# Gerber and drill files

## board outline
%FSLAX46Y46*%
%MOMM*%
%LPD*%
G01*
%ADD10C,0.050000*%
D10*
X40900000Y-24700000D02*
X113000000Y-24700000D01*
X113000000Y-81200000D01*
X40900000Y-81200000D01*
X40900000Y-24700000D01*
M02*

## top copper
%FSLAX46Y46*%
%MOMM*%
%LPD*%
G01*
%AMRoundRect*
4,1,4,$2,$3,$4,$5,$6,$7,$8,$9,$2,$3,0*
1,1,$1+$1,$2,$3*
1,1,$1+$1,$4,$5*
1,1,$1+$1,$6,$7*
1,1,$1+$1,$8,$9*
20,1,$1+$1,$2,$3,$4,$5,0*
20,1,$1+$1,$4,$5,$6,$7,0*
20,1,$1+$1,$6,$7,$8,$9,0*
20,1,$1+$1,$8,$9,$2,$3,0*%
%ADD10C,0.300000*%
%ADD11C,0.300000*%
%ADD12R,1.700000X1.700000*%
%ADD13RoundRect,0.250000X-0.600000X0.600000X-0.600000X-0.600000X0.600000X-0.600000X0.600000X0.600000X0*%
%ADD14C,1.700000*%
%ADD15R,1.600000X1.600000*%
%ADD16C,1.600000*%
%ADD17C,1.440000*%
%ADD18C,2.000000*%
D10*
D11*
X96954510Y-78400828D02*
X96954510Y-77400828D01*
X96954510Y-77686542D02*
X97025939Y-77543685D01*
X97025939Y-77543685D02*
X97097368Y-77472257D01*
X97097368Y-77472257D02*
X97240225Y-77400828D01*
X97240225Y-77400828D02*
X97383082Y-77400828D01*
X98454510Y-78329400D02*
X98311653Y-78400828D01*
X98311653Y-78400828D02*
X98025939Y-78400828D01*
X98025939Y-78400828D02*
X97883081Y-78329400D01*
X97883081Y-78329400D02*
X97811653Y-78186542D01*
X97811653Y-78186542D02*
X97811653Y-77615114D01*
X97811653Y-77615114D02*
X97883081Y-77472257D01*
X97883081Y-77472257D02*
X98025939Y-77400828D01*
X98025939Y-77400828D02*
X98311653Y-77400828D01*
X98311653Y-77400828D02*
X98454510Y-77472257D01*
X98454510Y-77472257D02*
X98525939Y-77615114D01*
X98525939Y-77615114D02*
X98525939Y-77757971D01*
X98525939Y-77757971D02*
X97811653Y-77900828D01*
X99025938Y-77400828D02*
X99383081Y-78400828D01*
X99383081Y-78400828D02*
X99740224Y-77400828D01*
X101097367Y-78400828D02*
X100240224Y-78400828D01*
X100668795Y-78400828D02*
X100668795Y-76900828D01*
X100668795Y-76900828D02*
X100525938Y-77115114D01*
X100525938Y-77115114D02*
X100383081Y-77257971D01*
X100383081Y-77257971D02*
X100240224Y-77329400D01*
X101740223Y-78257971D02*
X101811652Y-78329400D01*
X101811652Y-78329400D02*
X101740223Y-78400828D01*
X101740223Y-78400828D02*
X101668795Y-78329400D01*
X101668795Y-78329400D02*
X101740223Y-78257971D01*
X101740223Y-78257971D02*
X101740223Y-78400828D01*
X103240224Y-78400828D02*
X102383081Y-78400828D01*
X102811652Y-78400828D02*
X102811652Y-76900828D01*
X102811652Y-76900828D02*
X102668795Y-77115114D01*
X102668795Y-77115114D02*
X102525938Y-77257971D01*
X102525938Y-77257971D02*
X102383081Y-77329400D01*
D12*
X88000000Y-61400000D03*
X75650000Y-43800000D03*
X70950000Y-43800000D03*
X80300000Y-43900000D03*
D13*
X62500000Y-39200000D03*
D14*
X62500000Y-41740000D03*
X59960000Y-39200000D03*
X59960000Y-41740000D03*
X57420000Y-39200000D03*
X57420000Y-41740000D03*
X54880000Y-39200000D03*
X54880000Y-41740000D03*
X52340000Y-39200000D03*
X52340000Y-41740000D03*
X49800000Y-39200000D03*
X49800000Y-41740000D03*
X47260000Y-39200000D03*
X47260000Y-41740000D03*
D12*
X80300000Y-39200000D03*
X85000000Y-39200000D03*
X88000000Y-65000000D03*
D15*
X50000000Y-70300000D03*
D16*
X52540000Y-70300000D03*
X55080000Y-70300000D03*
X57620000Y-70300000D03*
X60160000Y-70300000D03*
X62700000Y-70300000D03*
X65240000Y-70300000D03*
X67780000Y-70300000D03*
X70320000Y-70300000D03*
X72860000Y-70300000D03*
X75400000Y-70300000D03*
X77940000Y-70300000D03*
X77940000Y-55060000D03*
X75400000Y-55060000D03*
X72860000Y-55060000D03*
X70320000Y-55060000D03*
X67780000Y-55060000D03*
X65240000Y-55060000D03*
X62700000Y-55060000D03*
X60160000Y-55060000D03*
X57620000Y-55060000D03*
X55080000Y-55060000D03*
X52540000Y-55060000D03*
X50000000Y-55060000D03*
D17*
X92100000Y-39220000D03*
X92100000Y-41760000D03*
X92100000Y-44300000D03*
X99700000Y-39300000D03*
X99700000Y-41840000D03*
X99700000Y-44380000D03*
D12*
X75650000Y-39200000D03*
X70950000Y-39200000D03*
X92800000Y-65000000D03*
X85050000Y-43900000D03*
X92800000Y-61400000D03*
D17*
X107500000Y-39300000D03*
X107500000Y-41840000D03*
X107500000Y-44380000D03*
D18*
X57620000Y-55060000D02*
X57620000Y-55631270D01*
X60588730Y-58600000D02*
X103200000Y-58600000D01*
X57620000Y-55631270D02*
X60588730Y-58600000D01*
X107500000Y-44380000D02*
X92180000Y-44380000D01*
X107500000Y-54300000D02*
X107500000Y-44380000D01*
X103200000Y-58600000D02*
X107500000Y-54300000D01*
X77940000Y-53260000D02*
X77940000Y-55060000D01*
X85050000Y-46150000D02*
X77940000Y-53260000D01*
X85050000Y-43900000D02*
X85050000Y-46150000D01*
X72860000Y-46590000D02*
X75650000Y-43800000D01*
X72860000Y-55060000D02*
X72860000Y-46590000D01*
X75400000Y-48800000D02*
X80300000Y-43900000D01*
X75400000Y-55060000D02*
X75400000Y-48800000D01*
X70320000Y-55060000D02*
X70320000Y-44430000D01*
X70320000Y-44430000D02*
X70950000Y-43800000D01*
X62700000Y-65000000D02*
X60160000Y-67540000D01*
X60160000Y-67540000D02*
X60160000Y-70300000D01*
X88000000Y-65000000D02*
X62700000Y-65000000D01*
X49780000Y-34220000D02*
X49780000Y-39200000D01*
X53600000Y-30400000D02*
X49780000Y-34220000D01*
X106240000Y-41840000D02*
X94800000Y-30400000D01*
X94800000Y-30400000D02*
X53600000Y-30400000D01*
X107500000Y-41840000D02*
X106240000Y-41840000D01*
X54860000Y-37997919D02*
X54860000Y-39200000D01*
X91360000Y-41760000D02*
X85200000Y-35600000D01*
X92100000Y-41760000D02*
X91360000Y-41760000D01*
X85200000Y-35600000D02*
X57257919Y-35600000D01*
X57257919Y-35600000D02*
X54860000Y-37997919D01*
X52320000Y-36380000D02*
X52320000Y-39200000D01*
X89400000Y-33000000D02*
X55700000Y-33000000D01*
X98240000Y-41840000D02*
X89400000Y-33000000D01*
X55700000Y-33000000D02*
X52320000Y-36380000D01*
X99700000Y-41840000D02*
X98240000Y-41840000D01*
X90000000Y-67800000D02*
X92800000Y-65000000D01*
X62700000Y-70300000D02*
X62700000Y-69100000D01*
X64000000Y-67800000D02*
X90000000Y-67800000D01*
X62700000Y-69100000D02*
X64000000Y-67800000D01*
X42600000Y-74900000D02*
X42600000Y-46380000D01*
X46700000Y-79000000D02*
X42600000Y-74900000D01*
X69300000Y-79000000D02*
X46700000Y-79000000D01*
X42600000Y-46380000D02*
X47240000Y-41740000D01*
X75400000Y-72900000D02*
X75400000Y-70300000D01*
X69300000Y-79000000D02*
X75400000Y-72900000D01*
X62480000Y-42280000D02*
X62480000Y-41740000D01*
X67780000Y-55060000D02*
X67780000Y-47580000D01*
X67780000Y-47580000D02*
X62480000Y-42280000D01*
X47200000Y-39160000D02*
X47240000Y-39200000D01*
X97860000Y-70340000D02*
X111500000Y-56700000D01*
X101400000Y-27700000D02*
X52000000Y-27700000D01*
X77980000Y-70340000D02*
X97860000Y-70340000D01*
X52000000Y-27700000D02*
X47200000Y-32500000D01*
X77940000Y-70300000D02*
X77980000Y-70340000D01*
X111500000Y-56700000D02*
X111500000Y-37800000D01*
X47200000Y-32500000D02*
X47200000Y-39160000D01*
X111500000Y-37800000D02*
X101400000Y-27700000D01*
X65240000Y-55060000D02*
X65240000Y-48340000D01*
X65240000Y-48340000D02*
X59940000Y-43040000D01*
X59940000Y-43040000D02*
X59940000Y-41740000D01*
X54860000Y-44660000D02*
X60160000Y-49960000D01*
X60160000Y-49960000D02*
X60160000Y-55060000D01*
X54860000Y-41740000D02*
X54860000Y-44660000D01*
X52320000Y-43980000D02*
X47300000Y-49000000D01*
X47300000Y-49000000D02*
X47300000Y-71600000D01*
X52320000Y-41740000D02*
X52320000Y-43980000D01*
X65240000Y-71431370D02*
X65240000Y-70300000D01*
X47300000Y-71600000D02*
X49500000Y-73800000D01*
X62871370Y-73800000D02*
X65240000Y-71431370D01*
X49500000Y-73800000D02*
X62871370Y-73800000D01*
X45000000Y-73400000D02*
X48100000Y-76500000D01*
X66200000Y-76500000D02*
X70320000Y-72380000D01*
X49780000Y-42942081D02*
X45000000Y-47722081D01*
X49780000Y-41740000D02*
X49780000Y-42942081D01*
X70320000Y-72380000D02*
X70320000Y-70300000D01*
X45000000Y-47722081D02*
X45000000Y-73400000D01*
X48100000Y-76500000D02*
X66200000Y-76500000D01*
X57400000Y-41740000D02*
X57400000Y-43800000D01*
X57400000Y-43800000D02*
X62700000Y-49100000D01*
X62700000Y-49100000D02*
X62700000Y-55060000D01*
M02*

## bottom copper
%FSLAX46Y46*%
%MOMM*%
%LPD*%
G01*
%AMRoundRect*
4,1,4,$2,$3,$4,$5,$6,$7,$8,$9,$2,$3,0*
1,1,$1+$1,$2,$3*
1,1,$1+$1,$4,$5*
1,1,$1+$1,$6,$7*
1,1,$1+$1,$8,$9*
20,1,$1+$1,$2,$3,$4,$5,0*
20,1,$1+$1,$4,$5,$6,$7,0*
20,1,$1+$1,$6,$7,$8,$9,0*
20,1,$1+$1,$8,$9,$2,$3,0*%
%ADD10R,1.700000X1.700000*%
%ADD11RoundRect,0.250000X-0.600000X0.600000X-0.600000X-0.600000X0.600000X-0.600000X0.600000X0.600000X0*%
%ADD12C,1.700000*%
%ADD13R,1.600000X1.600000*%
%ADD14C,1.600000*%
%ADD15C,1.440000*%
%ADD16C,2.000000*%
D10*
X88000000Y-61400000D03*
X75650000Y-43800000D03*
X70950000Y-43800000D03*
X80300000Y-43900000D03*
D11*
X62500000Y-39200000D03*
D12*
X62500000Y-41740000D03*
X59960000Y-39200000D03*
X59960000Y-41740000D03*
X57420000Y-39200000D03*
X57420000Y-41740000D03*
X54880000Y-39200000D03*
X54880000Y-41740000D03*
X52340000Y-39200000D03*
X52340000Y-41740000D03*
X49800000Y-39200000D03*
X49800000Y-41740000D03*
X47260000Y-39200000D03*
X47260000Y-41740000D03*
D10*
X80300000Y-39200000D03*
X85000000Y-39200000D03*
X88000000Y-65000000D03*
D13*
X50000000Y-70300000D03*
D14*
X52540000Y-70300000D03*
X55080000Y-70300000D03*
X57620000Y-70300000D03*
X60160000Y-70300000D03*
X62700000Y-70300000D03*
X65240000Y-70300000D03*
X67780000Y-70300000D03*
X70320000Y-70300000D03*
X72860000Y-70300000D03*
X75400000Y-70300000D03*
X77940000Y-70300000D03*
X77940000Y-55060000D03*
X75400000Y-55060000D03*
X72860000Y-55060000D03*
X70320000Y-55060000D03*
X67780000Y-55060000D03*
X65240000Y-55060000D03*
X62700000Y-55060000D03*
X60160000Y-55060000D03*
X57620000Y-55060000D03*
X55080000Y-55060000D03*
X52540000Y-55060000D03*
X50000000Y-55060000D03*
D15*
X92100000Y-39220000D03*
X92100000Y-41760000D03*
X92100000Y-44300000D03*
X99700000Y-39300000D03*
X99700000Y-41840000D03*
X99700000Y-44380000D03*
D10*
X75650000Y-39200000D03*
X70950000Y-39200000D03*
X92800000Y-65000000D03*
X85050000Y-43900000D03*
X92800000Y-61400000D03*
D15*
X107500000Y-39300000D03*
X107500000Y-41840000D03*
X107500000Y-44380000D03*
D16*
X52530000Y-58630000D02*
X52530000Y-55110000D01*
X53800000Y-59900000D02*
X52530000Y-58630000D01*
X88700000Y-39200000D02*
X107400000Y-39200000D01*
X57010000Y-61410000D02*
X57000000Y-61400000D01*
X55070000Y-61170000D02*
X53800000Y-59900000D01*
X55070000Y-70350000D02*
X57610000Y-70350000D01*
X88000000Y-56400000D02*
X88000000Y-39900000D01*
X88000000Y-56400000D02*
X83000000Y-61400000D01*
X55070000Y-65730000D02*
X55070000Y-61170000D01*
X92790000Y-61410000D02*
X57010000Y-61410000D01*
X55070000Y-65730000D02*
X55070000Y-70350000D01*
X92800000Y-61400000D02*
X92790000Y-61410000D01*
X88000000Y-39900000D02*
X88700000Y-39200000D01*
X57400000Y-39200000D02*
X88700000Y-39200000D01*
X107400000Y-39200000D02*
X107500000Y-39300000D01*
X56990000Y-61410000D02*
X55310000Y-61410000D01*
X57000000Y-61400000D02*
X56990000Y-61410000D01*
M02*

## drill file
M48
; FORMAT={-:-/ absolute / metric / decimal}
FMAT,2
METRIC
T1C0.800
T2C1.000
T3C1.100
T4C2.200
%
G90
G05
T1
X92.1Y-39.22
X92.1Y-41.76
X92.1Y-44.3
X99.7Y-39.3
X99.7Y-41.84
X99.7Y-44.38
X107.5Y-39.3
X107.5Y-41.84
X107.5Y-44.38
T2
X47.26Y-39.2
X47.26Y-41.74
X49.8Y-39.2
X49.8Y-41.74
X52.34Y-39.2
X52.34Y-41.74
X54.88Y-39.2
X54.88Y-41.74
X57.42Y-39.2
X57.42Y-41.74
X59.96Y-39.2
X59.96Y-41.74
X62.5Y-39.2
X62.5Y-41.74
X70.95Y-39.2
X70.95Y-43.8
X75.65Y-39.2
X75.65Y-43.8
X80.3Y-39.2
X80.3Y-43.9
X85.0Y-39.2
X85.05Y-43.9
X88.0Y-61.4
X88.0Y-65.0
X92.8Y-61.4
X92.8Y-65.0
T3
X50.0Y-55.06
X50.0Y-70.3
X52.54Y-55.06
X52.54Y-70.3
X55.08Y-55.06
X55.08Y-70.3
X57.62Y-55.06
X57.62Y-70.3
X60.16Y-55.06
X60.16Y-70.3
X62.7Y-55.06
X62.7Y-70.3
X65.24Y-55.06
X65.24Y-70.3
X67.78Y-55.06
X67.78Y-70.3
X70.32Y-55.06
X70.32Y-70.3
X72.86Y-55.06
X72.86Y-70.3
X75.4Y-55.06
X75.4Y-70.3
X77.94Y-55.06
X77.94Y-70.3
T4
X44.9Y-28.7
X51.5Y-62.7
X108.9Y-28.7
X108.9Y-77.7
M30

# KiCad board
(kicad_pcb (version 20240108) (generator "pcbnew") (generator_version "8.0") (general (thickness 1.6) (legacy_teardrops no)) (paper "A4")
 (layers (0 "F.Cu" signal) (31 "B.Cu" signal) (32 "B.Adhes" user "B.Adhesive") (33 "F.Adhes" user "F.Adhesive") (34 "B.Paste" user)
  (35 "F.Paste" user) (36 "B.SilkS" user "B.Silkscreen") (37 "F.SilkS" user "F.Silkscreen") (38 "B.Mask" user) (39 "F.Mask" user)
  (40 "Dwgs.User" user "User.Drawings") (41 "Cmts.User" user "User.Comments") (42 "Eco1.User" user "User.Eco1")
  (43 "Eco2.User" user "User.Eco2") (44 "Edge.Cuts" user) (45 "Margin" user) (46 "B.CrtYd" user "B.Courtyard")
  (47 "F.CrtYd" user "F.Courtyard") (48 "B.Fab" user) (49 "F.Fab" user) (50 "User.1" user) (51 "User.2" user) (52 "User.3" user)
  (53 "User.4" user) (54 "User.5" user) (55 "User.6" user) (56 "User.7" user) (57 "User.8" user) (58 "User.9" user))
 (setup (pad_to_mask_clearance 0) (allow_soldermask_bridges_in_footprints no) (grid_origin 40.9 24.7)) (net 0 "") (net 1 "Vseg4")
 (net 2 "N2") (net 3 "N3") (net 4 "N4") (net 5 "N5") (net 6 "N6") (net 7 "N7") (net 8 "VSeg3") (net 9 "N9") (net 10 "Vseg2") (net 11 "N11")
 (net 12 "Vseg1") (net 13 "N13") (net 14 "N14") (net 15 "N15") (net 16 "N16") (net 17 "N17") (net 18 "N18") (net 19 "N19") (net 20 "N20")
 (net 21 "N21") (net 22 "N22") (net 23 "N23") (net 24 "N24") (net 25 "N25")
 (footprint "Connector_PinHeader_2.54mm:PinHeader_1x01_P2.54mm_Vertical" (layer "F.Cu") (at 88 61.4 -90)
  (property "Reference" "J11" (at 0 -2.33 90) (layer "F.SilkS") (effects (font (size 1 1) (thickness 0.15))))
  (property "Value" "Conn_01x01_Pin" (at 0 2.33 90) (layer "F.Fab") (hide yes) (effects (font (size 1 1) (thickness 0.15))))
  (pad "1" thru_hole rect (at 0 0 270) (size 1.7 1.7) (drill 1) (layers "*.Cu" "*.Mask") (remove_unused_layers no) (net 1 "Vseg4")))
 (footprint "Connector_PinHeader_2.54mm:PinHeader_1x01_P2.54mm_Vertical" (layer "F.Cu") (at 75.65 43.8 180)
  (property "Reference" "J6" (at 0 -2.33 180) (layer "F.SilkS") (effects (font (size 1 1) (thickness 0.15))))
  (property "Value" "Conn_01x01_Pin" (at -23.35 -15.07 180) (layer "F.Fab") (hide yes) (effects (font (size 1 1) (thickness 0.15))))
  (pad "1" thru_hole rect (at 0 0 180) (size 1.7 1.7) (drill 1) (layers "*.Cu" "*.Mask") (remove_unused_layers no) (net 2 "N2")))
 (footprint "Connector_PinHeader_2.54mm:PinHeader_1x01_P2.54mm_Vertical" (layer "F.Cu") (at 70.95 43.8 180)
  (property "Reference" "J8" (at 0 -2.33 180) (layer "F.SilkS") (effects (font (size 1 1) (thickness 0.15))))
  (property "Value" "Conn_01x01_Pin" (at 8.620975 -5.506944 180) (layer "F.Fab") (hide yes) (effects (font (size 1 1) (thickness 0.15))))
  (pad "1" thru_hole rect (at 0 0 180) (size 1.7 1.7) (drill 1) (layers "*.Cu" "*.Mask") (remove_unused_layers no) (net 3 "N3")))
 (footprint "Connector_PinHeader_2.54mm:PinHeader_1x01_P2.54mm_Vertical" (layer "F.Cu") (at 80.3 43.9 180)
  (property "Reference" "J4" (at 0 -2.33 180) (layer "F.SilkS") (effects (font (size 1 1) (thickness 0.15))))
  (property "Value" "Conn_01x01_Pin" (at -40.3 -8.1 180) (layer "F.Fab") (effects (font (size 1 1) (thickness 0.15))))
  (pad "1" thru_hole rect (at 0 0 180) (size 1.7 1.7) (drill 1) (layers "*.Cu" "*.Mask") (remove_unused_layers no) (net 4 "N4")))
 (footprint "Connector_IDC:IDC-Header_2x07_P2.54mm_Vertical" (layer "F.Cu") (at 62.5 39.2 -90)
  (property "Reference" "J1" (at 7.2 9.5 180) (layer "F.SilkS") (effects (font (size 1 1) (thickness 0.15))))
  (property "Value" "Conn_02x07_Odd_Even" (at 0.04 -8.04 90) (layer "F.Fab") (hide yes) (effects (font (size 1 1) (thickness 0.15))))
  (pad "1" thru_hole roundrect (at 0 0 270) (size 1.7 1.7) (drill 1) (layers "*.Cu" "*.Mask") (remove_unused_layers no)
   (roundrect_rratio 0.147059) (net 1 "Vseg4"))
  (pad "2" thru_hole circle (at 2.54 0 270) (size 1.7 1.7) (drill 1) (layers "*.Cu" "*.Mask") (remove_unused_layers no) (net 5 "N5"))
  (pad "3" thru_hole circle (at 0 2.54 270) (size 1.7 1.7) (drill 1) (layers "*.Cu" "*.Mask") (remove_unused_layers no) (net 1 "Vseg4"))
  (pad "4" thru_hole circle (at 2.54 2.54 270) (size 1.7 1.7) (drill 1) (layers "*.Cu" "*.Mask") (remove_unused_layers no) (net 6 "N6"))
  (pad "5" thru_hole circle (at 0 5.08 270) (size 1.7 1.7) (drill 1) (layers "*.Cu" "*.Mask") (remove_unused_layers no) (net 1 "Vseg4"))
  (pad "6" thru_hole circle (at 2.54 5.08 270) (size 1.7 1.7) (drill 1) (layers "*.Cu" "*.Mask") (remove_unused_layers no) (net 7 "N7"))
  (pad "7" thru_hole circle (at 0 7.62 270) (size 1.7 1.7) (drill 1) (layers "*.Cu" "*.Mask") (remove_unused_layers no) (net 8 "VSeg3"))
  (pad "8" thru_hole circle (at 2.54 7.62 270) (size 1.7 1.7) (drill 1) (layers "*.Cu" "*.Mask") (remove_unused_layers no) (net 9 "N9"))
  (pad "9" thru_hole circle (at 0 10.16 270) (size 1.7 1.7) (drill 1) (layers "*.Cu" "*.Mask") (remove_unused_layers no) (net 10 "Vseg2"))
  (pad "10" thru_hole circle (at 2.54 10.16 270) (size 1.7 1.7) (drill 1) (layers "*.Cu" "*.Mask") (remove_unused_layers no) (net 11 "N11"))
  (pad "11" thru_hole circle (at 0 12.7 270) (size 1.7 1.7) (drill 1) (layers "*.Cu" "*.Mask") (remove_unused_layers no) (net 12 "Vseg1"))
  (pad "12" thru_hole circle (at 2.54 12.7 270) (size 1.7 1.7) (drill 1) (layers "*.Cu" "*.Mask") (remove_unused_layers no) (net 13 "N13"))
  (pad "13" thru_hole circle (at 0 15.24 270) (size 1.7 1.7) (drill 1) (layers "*.Cu" "*.Mask") (remove_unused_layers no) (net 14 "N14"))
  (pad "14" thru_hole circle (at 2.54 15.24 270) (size 1.7 1.7) (drill 1) (layers "*.Cu" "*.Mask") (remove_unused_layers no) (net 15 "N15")))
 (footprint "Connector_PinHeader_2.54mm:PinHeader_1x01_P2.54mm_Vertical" (layer "F.Cu") (at 80.3 39.2 180)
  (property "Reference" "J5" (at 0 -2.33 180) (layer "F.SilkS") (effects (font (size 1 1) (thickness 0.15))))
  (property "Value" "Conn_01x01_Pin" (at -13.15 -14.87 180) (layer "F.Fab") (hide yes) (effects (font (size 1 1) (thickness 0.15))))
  (pad "1" thru_hole rect (at 0 0 180) (size 1.7 1.7) (drill 1) (layers "*.Cu" "*.Mask") (remove_unused_layers no) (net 1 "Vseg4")))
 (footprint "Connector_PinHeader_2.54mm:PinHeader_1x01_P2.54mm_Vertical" (layer "F.Cu") (at 85 39.2 180)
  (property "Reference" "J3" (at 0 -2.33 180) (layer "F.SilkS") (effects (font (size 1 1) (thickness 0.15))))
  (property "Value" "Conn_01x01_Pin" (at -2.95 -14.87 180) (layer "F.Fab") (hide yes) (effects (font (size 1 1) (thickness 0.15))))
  (pad "1" thru_hole rect (at 0 0 180) (size 1.7 1.7) (drill 1) (layers "*.Cu" "*.Mask") (remove_unused_layers no) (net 1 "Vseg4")))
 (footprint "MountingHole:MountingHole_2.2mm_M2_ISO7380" (layer "F.Cu") (at 51.5 62.7)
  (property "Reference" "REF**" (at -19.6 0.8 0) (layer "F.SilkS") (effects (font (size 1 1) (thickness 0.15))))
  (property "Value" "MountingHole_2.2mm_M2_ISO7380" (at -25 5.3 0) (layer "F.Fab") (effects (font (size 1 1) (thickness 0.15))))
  (pad "" np_thru_hole circle (at 0 0) (size 2.2 2.2) (drill 2.2) (layers "*.Cu" "*.Mask")))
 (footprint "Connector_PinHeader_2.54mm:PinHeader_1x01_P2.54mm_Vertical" (layer "F.Cu") (at 88 65 -90)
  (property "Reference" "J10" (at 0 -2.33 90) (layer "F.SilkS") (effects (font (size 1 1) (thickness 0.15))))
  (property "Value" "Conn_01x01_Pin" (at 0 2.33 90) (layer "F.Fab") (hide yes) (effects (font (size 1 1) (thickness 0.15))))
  (pad "1" thru_hole rect (at 0 0 270) (size 1.7 1.7) (drill 1) (layers "*.Cu" "*.Mask") (remove_unused_layers no) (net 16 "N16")))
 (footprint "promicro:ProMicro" (layer "F.Cu") (at 63.97 62.68)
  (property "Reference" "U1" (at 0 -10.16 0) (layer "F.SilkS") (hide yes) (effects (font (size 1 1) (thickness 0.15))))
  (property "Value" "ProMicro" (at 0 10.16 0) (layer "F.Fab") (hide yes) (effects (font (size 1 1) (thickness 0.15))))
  (pad "1" thru_hole rect (at -13.97 7.62) (size 1.6 1.6) (drill 1.1) (layers "*.Cu" "*.Mask" "F.SilkS") (remove_unused_layers no)
   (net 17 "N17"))
  (pad "2" thru_hole circle (at -11.43 7.62) (size 1.6 1.6) (drill 1.1) (layers "*.Cu" "*.Mask" "F.SilkS") (remove_unused_layers no)
   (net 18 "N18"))
  (pad "3" thru_hole circle (at -8.89 7.62) (size 1.6 1.6) (drill 1.1) (layers "*.Cu" "*.Mask" "F.SilkS") (remove_unused_layers no)
   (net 1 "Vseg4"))
  (pad "4" thru_hole circle (at -6.35 7.62) (size 1.6 1.6) (drill 1.1) (layers "*.Cu" "*.Mask" "F.SilkS") (remove_unused_layers no)
   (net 1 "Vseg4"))
  (pad "5" thru_hole circle (at -3.81 7.62) (size 1.6 1.6) (drill 1.1) (layers "*.Cu" "*.Mask" "F.SilkS") (remove_unused_layers no)
   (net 16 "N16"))
  (pad "6" thru_hole circle (at -1.27 7.62) (size 1.6 1.6) (drill 1.1) (layers "*.Cu" "*.Mask" "F.SilkS") (remove_unused_layers no)
   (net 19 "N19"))
  (pad "7" thru_hole circle (at 1.27 7.62) (size 1.6 1.6) (drill 1.1) (layers "*.Cu" "*.Mask" "F.SilkS") (remove_unused_layers no)
   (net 11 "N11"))
  (pad "8" thru_hole circle (at 3.81 7.62) (size 1.6 1.6) (drill 1.1) (layers "*.Cu" "*.Mask" "F.SilkS") (remove_unused_layers no)
   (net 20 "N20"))
  (pad "9" thru_hole circle (at 6.35 7.62) (size 1.6 1.6) (drill 1.1) (layers "*.Cu" "*.Mask" "F.SilkS") (remove_unused_layers no)
   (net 13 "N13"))
  (pad "10" thru_hole circle (at 8.89 7.62) (size 1.6 1.6) (drill 1.1) (layers "*.Cu" "*.Mask" "F.SilkS") (remove_unused_layers no)
   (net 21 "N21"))
  (pad "11" thru_hole circle (at 11.43 7.62) (size 1.6 1.6) (drill 1.1) (layers "*.Cu" "*.Mask" "F.SilkS") (remove_unused_layers no)
   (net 15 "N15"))
  (pad "12" thru_hole circle (at 13.97 7.62) (size 1.6 1.6) (drill 1.1) (layers "*.Cu" "*.Mask" "F.SilkS") (remove_unused_layers no)
   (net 14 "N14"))
  (pad "13" thru_hole circle (at 13.97 -7.62) (size 1.6 1.6) (drill 1.1) (layers "*.Cu" "*.Mask" "F.SilkS") (remove_unused_layers no)
   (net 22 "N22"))
  (pad "14" thru_hole circle (at 11.43 -7.62) (size 1.6 1.6) (drill 1.1) (layers "*.Cu" "*.Mask" "F.SilkS") (remove_unused_layers no)
   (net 4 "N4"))
  (pad "15" thru_hole circle (at 8.89 -7.62) (size 1.6 1.6) (drill 1.1) (layers "*.Cu" "*.Mask" "F.SilkS") (remove_unused_layers no)
   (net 2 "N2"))
  (pad "16" thru_hole circle (at 6.35 -7.62) (size 1.6 1.6) (drill 1.1) (layers "*.Cu" "*.Mask" "F.SilkS") (remove_unused_layers no)
   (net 3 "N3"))
  (pad "17" thru_hole circle (at 3.81 -7.62) (size 1.6 1.6) (drill 1.1) (layers "*.Cu" "*.Mask" "F.SilkS") (remove_unused_layers no)
   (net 5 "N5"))
  (pad "18" thru_hole circle (at 1.27 -7.62) (size 1.6 1.6) (drill 1.1) (layers "*.Cu" "*.Mask" "F.SilkS") (remove_unused_layers no)
   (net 6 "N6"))
  (pad "19" thru_hole circle (at -1.27 -7.62) (size 1.6 1.6) (drill 1.1) (layers "*.Cu" "*.Mask" "F.SilkS") (remove_unused_layers no)
   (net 7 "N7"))
  (pad "20" thru_hole circle (at -3.81 -7.62) (size 1.6 1.6) (drill 1.1) (layers "*.Cu" "*.Mask" "F.SilkS") (remove_unused_layers no)
   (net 9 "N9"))
  (pad "21" thru_hole circle (at -6.35 -7.62) (size 1.6 1.6) (drill 1.1) (layers "*.Cu" "*.Mask" "F.SilkS") (remove_unused_layers no)
   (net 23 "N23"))
  (pad "22" thru_hole circle (at -8.89 -7.62) (size 1.6 1.6) (drill 1.1) (layers "*.Cu" "*.Mask" "F.SilkS") (remove_unused_layers no)
   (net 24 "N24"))
  (pad "23" thru_hole circle (at -11.43 -7.62) (size 1.6 1.6) (drill 1.1) (layers "*.Cu" "*.Mask" "F.SilkS") (remove_unused_layers no)
   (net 1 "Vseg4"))
  (pad "24" thru_hole circle (at -13.97 -7.62) (size 1.6 1.6) (drill 1.1) (layers "*.Cu" "*.Mask" "F.SilkS") (remove_unused_layers no)
   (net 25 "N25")))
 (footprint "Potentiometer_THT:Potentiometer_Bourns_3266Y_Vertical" (layer "F.Cu") (at 92.1 39.22 90)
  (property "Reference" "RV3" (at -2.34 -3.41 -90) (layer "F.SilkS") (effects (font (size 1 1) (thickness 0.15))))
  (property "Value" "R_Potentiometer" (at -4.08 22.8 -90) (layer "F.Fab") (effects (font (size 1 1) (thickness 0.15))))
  (pad "1" thru_hole circle (at 0 0 90) (size 1.44 1.44) (drill 0.8) (layers "*.Cu" "*.Mask") (remove_unused_layers no) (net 1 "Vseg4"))
  (pad "2" thru_hole circle (at -2.54 0 90) (size 1.44 1.44) (drill 0.8) (layers "*.Cu" "*.Mask") (remove_unused_layers no) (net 8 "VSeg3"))
  (pad "3" thru_hole circle (at -5.08 0 90) (size 1.44 1.44) (drill 0.8) (layers "*.Cu" "*.Mask") (remove_unused_layers no) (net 23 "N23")))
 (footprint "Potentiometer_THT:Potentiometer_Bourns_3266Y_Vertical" (layer "F.Cu") (at 99.7 39.3 90)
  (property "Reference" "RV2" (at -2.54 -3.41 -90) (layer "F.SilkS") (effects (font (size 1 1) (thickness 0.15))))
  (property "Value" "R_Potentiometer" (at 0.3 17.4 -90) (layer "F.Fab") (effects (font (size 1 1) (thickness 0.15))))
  (pad "1" thru_hole circle (at 0 0 90) (size 1.44 1.44) (drill 0.8) (layers "*.Cu" "*.Mask") (remove_unused_layers no) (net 1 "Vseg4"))
  (pad "2" thru_hole circle (at -2.54 0 90) (size 1.44 1.44) (drill 0.8) (layers "*.Cu" "*.Mask") (remove_unused_layers no) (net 10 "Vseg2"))
  (pad "3" thru_hole circle (at -5.08 0 90) (size 1.44 1.44) (drill 0.8) (layers "*.Cu" "*.Mask") (remove_unused_layers no) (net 23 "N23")))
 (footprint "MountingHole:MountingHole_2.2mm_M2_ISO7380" (layer "F.Cu") (at 108.9 77.7)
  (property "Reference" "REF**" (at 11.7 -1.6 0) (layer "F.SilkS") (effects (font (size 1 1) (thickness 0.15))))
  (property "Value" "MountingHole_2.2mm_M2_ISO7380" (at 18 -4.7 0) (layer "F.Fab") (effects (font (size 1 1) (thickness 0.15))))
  (pad "" np_thru_hole circle (at 0 0) (size 2.2 2.2) (drill 2.2) (layers "F&B.Cu" "*.Mask")))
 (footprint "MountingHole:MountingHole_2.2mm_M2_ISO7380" (layer "F.Cu") (at 44.9 28.7)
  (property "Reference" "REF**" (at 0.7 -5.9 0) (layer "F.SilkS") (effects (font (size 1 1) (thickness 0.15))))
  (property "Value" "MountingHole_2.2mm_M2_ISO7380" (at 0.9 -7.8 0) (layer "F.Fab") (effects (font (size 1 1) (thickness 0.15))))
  (pad "" np_thru_hole circle (at 0 0) (size 2.2 2.2) (drill 2.2) (layers "*.Cu" "*.Mask")))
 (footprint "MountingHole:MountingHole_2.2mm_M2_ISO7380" (layer "F.Cu") (at 108.9 28.7)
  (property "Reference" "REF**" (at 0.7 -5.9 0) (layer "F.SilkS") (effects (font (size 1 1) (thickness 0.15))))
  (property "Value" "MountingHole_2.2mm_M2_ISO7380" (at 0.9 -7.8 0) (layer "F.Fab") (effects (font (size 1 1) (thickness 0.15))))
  (pad "" np_thru_hole circle (at 0 0) (size 2.2 2.2) (drill 2.2) (layers "F&B.Cu" "*.Mask")))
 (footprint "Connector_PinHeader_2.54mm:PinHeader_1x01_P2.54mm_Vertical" (layer "F.Cu") (at 75.65 39.2 180)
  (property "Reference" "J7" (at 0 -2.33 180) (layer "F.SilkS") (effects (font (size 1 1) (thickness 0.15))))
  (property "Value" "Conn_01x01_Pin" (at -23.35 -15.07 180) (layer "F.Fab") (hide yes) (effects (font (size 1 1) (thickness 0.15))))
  (pad "1" thru_hole rect (at 0 0 180) (size 1.7 1.7) (drill 1) (layers "*.Cu" "*.Mask") (remove_unused_layers no) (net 1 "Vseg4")))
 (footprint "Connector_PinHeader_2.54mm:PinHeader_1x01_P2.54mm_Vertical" (layer "F.Cu") (at 70.95 39.2 180)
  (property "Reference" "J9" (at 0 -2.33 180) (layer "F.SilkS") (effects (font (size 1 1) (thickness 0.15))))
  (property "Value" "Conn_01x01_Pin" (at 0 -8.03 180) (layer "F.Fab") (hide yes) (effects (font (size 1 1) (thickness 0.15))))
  (pad "1" thru_hole rect (at 0 0 180) (size 1.7 1.7) (drill 1) (layers "*.Cu" "*.Mask") (remove_unused_layers no) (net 1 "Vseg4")))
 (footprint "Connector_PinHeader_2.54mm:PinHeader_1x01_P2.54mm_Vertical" (layer "F.Cu") (at 92.8 65 -90)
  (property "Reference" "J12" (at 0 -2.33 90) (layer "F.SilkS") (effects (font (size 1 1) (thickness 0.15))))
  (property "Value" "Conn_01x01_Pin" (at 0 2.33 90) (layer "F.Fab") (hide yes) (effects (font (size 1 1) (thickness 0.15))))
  (pad "1" thru_hole rect (at 0 0 270) (size 1.7 1.7) (drill 1) (layers "*.Cu" "*.Mask") (remove_unused_layers no) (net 19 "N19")))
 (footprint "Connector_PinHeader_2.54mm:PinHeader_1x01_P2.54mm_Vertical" (layer "F.Cu") (at 85.05 43.9 180)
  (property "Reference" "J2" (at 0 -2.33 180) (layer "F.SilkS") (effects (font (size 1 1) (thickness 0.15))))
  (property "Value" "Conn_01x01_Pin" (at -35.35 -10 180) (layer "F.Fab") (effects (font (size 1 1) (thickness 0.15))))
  (pad "1" thru_hole rect (at 0 0 180) (size 1.7 1.7) (drill 1) (layers "*.Cu" "*.Mask") (remove_unused_layers no) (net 22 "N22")))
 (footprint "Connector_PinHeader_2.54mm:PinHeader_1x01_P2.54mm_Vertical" (layer "F.Cu") (at 92.8 61.4 -90)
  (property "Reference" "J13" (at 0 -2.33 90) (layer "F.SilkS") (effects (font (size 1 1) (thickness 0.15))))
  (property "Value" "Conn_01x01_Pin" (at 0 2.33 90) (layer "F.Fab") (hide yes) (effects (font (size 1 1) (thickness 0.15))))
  (pad "1" thru_hole rect (at 0 0 270) (size 1.7 1.7) (drill 1) (layers "*.Cu" "*.Mask") (remove_unused_layers no) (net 1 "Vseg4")))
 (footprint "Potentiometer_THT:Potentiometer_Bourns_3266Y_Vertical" (layer "F.Cu") (at 107.5 39.3 90)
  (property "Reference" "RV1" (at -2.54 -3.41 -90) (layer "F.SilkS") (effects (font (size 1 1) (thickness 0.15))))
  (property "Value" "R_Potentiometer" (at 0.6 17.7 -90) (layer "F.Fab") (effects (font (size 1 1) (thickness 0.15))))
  (pad "1" thru_hole circle (at 0 0 90) (size 1.44 1.44) (drill 0.8) (layers "*.Cu" "*.Mask") (remove_unused_layers no) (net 1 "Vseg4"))
  (pad "2" thru_hole circle (at -2.54 0 90) (size 1.44 1.44) (drill 0.8) (layers "*.Cu" "*.Mask") (remove_unused_layers no) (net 12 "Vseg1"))
  (pad "3" thru_hole circle (at -5.08 0 90) (size 1.44 1.44) (drill 0.8) (layers "*.Cu" "*.Mask") (remove_unused_layers no) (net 23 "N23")))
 (gr_rect (start 40.9 24.7) (end 113 81.2) (stroke (width 0.05) (type default)) (fill none) (layer "Edge.Cuts"))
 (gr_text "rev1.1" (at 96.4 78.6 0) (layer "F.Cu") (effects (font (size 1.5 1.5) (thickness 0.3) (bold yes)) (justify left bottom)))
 (segment (start 57.62 55.06) (end 57.62 55.63127) (width 2) (layer "F.Cu") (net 23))
 (segment (start 60.58873 58.6) (end 103.2 58.6) (width 2) (layer "F.Cu") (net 23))
 (segment (start 57.62 55.63127) (end 60.58873 58.6) (width 2) (layer "F.Cu") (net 23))
 (segment (start 107.5 44.38) (end 92.18 44.38) (width 2) (layer "F.Cu") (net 23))
 (segment (start 107.5 54.3) (end 107.5 44.38) (width 2) (layer "F.Cu") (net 23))
 (segment (start 103.2 58.6) (end 107.5 54.3) (width 2) (layer "F.Cu") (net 23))
 (segment (start 77.94 53.26) (end 77.94 55.06) (width 2) (layer "F.Cu") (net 22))
 (segment (start 85.05 46.15) (end 77.94 53.26) (width 2) (layer "F.Cu") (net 22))
 (segment (start 85.05 43.9) (end 85.05 46.15) (width 2) (layer "F.Cu") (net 22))
 (segment (start 72.86 46.59) (end 75.65 43.8) (width 2) (layer "F.Cu") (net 2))
 (segment (start 72.86 55.06) (end 72.86 46.59) (width 2) (layer "F.Cu") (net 2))
 (segment (start 75.4 48.8) (end 80.3 43.9) (width 2) (layer "F.Cu") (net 4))
 (segment (start 75.4 55.06) (end 75.4 48.8) (width 2) (layer "F.Cu") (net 4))
 (segment (start 70.32 55.06) (end 70.32 44.43) (width 2) (layer "F.Cu") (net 3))
 (segment (start 70.32 44.43) (end 70.95 43.8) (width 2) (layer "F.Cu") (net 3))
 (segment (start 62.7 65) (end 60.16 67.54) (width 2) (layer "F.Cu") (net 16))
 (segment (start 60.16 67.54) (end 60.16 70.3) (width 2) (layer "F.Cu") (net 16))
 (segment (start 88 65) (end 62.7 65) (width 2) (layer "F.Cu") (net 16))
 (segment (start 49.78 34.22) (end 49.78 39.2) (width 2) (layer "F.Cu") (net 12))
 (segment (start 53.6 30.4) (end 49.78 34.22) (width 2) (layer "F.Cu") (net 12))
 (segment (start 106.24 41.84) (end 94.8 30.4) (width 2) (layer "F.Cu") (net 12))
 (segment (start 94.8 30.4) (end 53.6 30.4) (width 2) (layer "F.Cu") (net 12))
 (segment (start 107.5 41.84) (end 106.24 41.84) (width 2) (layer "F.Cu") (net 12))
 (segment (start 54.86 37.997919) (end 54.86 39.2) (width 2) (layer "F.Cu") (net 8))
 (segment (start 91.36 41.76) (end 85.2 35.6) (width 2) (layer "F.Cu") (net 8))
 (segment (start 92.1 41.76) (end 91.36 41.76) (width 2) (layer "F.Cu") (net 8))
 (segment (start 85.2 35.6) (end 57.257919 35.6) (width 2) (layer "F.Cu") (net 8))
 (segment (start 57.257919 35.6) (end 54.86 37.997919) (width 2) (layer "F.Cu") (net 8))
 (segment (start 52.53 58.63) (end 52.53 55.11) (width 2) (layer "B.Cu") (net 1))
 (segment (start 53.8 59.9) (end 52.53 58.63) (width 2) (layer "B.Cu") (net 1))
 (segment (start 88.7 39.2) (end 107.4 39.2) (width 2) (layer "B.Cu") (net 1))
 (segment (start 57.01 61.41) (end 57 61.4) (width 2) (layer "B.Cu") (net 1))
 (segment (start 55.07 61.17) (end 53.8 59.9) (width 2) (layer "B.Cu") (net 1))
 (segment (start 55.07 70.35) (end 57.61 70.35) (width 2) (layer "B.Cu") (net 1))
 (segment (start 88 56.4) (end 88 39.9) (width 2) (layer "B.Cu") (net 1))
 (segment (start 88 56.4) (end 83 61.4) (width 2) (layer "B.Cu") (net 1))
 (segment (start 55.07 65.73) (end 55.07 61.17) (width 2) (layer "B.Cu") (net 1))
 (segment (start 92.79 61.41) (end 57.01 61.41) (width 2) (layer "B.Cu") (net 1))
 (segment (start 55.07 65.73) (end 55.07 70.35) (width 2) (layer "B.Cu") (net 1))
 (segment (start 92.8 61.4) (end 92.79 61.41) (width 2) (layer "B.Cu") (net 1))
 (segment (start 88 39.9) (end 88.7 39.2) (width 2) (layer "B.Cu") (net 1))
 (segment (start 57.4 39.2) (end 88.7 39.2) (width 2) (layer "B.Cu") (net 1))
 (segment (start 107.4 39.2) (end 107.5 39.3) (width 2) (layer "B.Cu") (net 1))
 (segment (start 56.99 61.41) (end 55.31 61.41) (width 2) (layer "B.Cu") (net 1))
 (segment (start 57 61.4) (end 56.99 61.41) (width 2) (layer "B.Cu") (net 1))
 (segment (start 52.32 36.38) (end 52.32 39.2) (width 2) (layer "F.Cu") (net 10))
 (segment (start 89.4 33) (end 55.7 33) (width 2) (layer "F.Cu") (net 10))
 (segment (start 98.24 41.84) (end 89.4 33) (width 2) (layer "F.Cu") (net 10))
 (segment (start 55.7 33) (end 52.32 36.38) (width 2) (layer "F.Cu") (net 10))
 (segment (start 99.7 41.84) (end 98.24 41.84) (width 2) (layer "F.Cu") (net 10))
 (segment (start 90 67.8) (end 92.8 65) (width 2) (layer "F.Cu") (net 19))
 (segment (start 62.7 70.3) (end 62.7 69.1) (width 2) (layer "F.Cu") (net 19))
 (segment (start 64 67.8) (end 90 67.8) (width 2) (layer "F.Cu") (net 19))
 (segment (start 62.7 69.1) (end 64 67.8) (width 2) (layer "F.Cu") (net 19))
 (segment (start 42.6 74.9) (end 42.6 46.38) (width 2) (layer "F.Cu") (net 15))
 (segment (start 46.7 79) (end 42.6 74.9) (width 2) (layer "F.Cu") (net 15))
 (segment (start 69.3 79) (end 46.7 79) (width 2) (layer "F.Cu") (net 15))
 (segment (start 42.6 46.38) (end 47.24 41.74) (width 2) (layer "F.Cu") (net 15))
 (segment (start 75.4 72.9) (end 75.4 70.3) (width 2) (layer "F.Cu") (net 15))
 (segment (start 69.3 79) (end 75.4 72.9) (width 2) (layer "F.Cu") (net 15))
 (segment (start 62.48 42.28) (end 62.48 41.74) (width 2) (layer "F.Cu") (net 5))
 (segment (start 67.78 55.06) (end 67.78 47.58) (width 2) (layer "F.Cu") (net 5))
 (segment (start 67.78 47.58) (end 62.48 42.28) (width 2) (layer "F.Cu") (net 5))
 (segment (start 47.2 39.16) (end 47.24 39.2) (width 2) (layer "F.Cu") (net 14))
 (segment (start 97.86 70.34) (end 111.5 56.7) (width 2) (layer "F.Cu") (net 14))
 (segment (start 101.4 27.7) (end 52 27.7) (width 2) (layer "F.Cu") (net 14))
 (segment (start 77.98 70.34) (end 97.86 70.34) (width 2) (layer "F.Cu") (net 14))
 (segment (start 52 27.7) (end 47.2 32.5) (width 2) (layer "F.Cu") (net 14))
 (segment (start 77.94 70.3) (end 77.98 70.34) (width 2) (layer "F.Cu") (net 14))
 (segment (start 111.5 56.7) (end 111.5 37.8) (width 2) (layer "F.Cu") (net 14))
 (segment (start 47.2 32.5) (end 47.2 39.16) (width 2) (layer "F.Cu") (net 14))
 (segment (start 111.5 37.8) (end 101.4 27.7) (width 2) (layer "F.Cu") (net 14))
 (segment (start 65.24 55.06) (end 65.24 48.34) (width 2) (layer "F.Cu") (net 6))
 (segment (start 65.24 48.34) (end 59.94 43.04) (width 2) (layer "F.Cu") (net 6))
 (segment (start 59.94 43.04) (end 59.94 41.74) (width 2) (layer "F.Cu") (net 6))
 (segment (start 54.86 44.66) (end 60.16 49.96) (width 2) (layer "F.Cu") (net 9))
 (segment (start 60.16 49.96) (end 60.16 55.06) (width 2) (layer "F.Cu") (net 9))
 (segment (start 54.86 41.74) (end 54.86 44.66) (width 2) (layer "F.Cu") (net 9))
 (segment (start 52.32 43.98) (end 47.3 49) (width 2) (layer "F.Cu") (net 11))
 (segment (start 47.3 49) (end 47.3 71.6) (width 2) (layer "F.Cu") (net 11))
 (segment (start 52.32 41.74) (end 52.32 43.98) (width 2) (layer "F.Cu") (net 11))
 (segment (start 65.24 71.43137) (end 65.24 70.3) (width 2) (layer "F.Cu") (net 11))
 (segment (start 47.3 71.6) (end 49.5 73.8) (width 2) (layer "F.Cu") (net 11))
 (segment (start 62.87137 73.8) (end 65.24 71.43137) (width 2) (layer "F.Cu") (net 11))
 (segment (start 49.5 73.8) (end 62.87137 73.8) (width 2) (layer "F.Cu") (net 11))
 (segment (start 45 73.4) (end 48.1 76.5) (width 2) (layer "F.Cu") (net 13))
 (segment (start 66.2 76.5) (end 70.32 72.38) (width 2) (layer "F.Cu") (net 13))
 (segment (start 49.78 42.942081) (end 45 47.722081) (width 2) (layer "F.Cu") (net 13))
 (segment (start 49.78 41.74) (end 49.78 42.942081) (width 2) (layer "F.Cu") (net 13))
 (segment (start 70.32 72.38) (end 70.32 70.3) (width 2) (layer "F.Cu") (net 13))
 (segment (start 45 47.722081) (end 45 73.4) (width 2) (layer "F.Cu") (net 13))
 (segment (start 48.1 76.5) (end 66.2 76.5) (width 2) (layer "F.Cu") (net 13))
 (segment (start 57.4 41.74) (end 57.4 43.8) (width 2) (layer "F.Cu") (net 7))
 (segment (start 57.4 43.8) (end 62.7 49.1) (width 2) (layer "F.Cu") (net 7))
 (segment (start 62.7 49.1) (end 62.7 55.06) (width 2) (layer "F.Cu") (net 7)))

